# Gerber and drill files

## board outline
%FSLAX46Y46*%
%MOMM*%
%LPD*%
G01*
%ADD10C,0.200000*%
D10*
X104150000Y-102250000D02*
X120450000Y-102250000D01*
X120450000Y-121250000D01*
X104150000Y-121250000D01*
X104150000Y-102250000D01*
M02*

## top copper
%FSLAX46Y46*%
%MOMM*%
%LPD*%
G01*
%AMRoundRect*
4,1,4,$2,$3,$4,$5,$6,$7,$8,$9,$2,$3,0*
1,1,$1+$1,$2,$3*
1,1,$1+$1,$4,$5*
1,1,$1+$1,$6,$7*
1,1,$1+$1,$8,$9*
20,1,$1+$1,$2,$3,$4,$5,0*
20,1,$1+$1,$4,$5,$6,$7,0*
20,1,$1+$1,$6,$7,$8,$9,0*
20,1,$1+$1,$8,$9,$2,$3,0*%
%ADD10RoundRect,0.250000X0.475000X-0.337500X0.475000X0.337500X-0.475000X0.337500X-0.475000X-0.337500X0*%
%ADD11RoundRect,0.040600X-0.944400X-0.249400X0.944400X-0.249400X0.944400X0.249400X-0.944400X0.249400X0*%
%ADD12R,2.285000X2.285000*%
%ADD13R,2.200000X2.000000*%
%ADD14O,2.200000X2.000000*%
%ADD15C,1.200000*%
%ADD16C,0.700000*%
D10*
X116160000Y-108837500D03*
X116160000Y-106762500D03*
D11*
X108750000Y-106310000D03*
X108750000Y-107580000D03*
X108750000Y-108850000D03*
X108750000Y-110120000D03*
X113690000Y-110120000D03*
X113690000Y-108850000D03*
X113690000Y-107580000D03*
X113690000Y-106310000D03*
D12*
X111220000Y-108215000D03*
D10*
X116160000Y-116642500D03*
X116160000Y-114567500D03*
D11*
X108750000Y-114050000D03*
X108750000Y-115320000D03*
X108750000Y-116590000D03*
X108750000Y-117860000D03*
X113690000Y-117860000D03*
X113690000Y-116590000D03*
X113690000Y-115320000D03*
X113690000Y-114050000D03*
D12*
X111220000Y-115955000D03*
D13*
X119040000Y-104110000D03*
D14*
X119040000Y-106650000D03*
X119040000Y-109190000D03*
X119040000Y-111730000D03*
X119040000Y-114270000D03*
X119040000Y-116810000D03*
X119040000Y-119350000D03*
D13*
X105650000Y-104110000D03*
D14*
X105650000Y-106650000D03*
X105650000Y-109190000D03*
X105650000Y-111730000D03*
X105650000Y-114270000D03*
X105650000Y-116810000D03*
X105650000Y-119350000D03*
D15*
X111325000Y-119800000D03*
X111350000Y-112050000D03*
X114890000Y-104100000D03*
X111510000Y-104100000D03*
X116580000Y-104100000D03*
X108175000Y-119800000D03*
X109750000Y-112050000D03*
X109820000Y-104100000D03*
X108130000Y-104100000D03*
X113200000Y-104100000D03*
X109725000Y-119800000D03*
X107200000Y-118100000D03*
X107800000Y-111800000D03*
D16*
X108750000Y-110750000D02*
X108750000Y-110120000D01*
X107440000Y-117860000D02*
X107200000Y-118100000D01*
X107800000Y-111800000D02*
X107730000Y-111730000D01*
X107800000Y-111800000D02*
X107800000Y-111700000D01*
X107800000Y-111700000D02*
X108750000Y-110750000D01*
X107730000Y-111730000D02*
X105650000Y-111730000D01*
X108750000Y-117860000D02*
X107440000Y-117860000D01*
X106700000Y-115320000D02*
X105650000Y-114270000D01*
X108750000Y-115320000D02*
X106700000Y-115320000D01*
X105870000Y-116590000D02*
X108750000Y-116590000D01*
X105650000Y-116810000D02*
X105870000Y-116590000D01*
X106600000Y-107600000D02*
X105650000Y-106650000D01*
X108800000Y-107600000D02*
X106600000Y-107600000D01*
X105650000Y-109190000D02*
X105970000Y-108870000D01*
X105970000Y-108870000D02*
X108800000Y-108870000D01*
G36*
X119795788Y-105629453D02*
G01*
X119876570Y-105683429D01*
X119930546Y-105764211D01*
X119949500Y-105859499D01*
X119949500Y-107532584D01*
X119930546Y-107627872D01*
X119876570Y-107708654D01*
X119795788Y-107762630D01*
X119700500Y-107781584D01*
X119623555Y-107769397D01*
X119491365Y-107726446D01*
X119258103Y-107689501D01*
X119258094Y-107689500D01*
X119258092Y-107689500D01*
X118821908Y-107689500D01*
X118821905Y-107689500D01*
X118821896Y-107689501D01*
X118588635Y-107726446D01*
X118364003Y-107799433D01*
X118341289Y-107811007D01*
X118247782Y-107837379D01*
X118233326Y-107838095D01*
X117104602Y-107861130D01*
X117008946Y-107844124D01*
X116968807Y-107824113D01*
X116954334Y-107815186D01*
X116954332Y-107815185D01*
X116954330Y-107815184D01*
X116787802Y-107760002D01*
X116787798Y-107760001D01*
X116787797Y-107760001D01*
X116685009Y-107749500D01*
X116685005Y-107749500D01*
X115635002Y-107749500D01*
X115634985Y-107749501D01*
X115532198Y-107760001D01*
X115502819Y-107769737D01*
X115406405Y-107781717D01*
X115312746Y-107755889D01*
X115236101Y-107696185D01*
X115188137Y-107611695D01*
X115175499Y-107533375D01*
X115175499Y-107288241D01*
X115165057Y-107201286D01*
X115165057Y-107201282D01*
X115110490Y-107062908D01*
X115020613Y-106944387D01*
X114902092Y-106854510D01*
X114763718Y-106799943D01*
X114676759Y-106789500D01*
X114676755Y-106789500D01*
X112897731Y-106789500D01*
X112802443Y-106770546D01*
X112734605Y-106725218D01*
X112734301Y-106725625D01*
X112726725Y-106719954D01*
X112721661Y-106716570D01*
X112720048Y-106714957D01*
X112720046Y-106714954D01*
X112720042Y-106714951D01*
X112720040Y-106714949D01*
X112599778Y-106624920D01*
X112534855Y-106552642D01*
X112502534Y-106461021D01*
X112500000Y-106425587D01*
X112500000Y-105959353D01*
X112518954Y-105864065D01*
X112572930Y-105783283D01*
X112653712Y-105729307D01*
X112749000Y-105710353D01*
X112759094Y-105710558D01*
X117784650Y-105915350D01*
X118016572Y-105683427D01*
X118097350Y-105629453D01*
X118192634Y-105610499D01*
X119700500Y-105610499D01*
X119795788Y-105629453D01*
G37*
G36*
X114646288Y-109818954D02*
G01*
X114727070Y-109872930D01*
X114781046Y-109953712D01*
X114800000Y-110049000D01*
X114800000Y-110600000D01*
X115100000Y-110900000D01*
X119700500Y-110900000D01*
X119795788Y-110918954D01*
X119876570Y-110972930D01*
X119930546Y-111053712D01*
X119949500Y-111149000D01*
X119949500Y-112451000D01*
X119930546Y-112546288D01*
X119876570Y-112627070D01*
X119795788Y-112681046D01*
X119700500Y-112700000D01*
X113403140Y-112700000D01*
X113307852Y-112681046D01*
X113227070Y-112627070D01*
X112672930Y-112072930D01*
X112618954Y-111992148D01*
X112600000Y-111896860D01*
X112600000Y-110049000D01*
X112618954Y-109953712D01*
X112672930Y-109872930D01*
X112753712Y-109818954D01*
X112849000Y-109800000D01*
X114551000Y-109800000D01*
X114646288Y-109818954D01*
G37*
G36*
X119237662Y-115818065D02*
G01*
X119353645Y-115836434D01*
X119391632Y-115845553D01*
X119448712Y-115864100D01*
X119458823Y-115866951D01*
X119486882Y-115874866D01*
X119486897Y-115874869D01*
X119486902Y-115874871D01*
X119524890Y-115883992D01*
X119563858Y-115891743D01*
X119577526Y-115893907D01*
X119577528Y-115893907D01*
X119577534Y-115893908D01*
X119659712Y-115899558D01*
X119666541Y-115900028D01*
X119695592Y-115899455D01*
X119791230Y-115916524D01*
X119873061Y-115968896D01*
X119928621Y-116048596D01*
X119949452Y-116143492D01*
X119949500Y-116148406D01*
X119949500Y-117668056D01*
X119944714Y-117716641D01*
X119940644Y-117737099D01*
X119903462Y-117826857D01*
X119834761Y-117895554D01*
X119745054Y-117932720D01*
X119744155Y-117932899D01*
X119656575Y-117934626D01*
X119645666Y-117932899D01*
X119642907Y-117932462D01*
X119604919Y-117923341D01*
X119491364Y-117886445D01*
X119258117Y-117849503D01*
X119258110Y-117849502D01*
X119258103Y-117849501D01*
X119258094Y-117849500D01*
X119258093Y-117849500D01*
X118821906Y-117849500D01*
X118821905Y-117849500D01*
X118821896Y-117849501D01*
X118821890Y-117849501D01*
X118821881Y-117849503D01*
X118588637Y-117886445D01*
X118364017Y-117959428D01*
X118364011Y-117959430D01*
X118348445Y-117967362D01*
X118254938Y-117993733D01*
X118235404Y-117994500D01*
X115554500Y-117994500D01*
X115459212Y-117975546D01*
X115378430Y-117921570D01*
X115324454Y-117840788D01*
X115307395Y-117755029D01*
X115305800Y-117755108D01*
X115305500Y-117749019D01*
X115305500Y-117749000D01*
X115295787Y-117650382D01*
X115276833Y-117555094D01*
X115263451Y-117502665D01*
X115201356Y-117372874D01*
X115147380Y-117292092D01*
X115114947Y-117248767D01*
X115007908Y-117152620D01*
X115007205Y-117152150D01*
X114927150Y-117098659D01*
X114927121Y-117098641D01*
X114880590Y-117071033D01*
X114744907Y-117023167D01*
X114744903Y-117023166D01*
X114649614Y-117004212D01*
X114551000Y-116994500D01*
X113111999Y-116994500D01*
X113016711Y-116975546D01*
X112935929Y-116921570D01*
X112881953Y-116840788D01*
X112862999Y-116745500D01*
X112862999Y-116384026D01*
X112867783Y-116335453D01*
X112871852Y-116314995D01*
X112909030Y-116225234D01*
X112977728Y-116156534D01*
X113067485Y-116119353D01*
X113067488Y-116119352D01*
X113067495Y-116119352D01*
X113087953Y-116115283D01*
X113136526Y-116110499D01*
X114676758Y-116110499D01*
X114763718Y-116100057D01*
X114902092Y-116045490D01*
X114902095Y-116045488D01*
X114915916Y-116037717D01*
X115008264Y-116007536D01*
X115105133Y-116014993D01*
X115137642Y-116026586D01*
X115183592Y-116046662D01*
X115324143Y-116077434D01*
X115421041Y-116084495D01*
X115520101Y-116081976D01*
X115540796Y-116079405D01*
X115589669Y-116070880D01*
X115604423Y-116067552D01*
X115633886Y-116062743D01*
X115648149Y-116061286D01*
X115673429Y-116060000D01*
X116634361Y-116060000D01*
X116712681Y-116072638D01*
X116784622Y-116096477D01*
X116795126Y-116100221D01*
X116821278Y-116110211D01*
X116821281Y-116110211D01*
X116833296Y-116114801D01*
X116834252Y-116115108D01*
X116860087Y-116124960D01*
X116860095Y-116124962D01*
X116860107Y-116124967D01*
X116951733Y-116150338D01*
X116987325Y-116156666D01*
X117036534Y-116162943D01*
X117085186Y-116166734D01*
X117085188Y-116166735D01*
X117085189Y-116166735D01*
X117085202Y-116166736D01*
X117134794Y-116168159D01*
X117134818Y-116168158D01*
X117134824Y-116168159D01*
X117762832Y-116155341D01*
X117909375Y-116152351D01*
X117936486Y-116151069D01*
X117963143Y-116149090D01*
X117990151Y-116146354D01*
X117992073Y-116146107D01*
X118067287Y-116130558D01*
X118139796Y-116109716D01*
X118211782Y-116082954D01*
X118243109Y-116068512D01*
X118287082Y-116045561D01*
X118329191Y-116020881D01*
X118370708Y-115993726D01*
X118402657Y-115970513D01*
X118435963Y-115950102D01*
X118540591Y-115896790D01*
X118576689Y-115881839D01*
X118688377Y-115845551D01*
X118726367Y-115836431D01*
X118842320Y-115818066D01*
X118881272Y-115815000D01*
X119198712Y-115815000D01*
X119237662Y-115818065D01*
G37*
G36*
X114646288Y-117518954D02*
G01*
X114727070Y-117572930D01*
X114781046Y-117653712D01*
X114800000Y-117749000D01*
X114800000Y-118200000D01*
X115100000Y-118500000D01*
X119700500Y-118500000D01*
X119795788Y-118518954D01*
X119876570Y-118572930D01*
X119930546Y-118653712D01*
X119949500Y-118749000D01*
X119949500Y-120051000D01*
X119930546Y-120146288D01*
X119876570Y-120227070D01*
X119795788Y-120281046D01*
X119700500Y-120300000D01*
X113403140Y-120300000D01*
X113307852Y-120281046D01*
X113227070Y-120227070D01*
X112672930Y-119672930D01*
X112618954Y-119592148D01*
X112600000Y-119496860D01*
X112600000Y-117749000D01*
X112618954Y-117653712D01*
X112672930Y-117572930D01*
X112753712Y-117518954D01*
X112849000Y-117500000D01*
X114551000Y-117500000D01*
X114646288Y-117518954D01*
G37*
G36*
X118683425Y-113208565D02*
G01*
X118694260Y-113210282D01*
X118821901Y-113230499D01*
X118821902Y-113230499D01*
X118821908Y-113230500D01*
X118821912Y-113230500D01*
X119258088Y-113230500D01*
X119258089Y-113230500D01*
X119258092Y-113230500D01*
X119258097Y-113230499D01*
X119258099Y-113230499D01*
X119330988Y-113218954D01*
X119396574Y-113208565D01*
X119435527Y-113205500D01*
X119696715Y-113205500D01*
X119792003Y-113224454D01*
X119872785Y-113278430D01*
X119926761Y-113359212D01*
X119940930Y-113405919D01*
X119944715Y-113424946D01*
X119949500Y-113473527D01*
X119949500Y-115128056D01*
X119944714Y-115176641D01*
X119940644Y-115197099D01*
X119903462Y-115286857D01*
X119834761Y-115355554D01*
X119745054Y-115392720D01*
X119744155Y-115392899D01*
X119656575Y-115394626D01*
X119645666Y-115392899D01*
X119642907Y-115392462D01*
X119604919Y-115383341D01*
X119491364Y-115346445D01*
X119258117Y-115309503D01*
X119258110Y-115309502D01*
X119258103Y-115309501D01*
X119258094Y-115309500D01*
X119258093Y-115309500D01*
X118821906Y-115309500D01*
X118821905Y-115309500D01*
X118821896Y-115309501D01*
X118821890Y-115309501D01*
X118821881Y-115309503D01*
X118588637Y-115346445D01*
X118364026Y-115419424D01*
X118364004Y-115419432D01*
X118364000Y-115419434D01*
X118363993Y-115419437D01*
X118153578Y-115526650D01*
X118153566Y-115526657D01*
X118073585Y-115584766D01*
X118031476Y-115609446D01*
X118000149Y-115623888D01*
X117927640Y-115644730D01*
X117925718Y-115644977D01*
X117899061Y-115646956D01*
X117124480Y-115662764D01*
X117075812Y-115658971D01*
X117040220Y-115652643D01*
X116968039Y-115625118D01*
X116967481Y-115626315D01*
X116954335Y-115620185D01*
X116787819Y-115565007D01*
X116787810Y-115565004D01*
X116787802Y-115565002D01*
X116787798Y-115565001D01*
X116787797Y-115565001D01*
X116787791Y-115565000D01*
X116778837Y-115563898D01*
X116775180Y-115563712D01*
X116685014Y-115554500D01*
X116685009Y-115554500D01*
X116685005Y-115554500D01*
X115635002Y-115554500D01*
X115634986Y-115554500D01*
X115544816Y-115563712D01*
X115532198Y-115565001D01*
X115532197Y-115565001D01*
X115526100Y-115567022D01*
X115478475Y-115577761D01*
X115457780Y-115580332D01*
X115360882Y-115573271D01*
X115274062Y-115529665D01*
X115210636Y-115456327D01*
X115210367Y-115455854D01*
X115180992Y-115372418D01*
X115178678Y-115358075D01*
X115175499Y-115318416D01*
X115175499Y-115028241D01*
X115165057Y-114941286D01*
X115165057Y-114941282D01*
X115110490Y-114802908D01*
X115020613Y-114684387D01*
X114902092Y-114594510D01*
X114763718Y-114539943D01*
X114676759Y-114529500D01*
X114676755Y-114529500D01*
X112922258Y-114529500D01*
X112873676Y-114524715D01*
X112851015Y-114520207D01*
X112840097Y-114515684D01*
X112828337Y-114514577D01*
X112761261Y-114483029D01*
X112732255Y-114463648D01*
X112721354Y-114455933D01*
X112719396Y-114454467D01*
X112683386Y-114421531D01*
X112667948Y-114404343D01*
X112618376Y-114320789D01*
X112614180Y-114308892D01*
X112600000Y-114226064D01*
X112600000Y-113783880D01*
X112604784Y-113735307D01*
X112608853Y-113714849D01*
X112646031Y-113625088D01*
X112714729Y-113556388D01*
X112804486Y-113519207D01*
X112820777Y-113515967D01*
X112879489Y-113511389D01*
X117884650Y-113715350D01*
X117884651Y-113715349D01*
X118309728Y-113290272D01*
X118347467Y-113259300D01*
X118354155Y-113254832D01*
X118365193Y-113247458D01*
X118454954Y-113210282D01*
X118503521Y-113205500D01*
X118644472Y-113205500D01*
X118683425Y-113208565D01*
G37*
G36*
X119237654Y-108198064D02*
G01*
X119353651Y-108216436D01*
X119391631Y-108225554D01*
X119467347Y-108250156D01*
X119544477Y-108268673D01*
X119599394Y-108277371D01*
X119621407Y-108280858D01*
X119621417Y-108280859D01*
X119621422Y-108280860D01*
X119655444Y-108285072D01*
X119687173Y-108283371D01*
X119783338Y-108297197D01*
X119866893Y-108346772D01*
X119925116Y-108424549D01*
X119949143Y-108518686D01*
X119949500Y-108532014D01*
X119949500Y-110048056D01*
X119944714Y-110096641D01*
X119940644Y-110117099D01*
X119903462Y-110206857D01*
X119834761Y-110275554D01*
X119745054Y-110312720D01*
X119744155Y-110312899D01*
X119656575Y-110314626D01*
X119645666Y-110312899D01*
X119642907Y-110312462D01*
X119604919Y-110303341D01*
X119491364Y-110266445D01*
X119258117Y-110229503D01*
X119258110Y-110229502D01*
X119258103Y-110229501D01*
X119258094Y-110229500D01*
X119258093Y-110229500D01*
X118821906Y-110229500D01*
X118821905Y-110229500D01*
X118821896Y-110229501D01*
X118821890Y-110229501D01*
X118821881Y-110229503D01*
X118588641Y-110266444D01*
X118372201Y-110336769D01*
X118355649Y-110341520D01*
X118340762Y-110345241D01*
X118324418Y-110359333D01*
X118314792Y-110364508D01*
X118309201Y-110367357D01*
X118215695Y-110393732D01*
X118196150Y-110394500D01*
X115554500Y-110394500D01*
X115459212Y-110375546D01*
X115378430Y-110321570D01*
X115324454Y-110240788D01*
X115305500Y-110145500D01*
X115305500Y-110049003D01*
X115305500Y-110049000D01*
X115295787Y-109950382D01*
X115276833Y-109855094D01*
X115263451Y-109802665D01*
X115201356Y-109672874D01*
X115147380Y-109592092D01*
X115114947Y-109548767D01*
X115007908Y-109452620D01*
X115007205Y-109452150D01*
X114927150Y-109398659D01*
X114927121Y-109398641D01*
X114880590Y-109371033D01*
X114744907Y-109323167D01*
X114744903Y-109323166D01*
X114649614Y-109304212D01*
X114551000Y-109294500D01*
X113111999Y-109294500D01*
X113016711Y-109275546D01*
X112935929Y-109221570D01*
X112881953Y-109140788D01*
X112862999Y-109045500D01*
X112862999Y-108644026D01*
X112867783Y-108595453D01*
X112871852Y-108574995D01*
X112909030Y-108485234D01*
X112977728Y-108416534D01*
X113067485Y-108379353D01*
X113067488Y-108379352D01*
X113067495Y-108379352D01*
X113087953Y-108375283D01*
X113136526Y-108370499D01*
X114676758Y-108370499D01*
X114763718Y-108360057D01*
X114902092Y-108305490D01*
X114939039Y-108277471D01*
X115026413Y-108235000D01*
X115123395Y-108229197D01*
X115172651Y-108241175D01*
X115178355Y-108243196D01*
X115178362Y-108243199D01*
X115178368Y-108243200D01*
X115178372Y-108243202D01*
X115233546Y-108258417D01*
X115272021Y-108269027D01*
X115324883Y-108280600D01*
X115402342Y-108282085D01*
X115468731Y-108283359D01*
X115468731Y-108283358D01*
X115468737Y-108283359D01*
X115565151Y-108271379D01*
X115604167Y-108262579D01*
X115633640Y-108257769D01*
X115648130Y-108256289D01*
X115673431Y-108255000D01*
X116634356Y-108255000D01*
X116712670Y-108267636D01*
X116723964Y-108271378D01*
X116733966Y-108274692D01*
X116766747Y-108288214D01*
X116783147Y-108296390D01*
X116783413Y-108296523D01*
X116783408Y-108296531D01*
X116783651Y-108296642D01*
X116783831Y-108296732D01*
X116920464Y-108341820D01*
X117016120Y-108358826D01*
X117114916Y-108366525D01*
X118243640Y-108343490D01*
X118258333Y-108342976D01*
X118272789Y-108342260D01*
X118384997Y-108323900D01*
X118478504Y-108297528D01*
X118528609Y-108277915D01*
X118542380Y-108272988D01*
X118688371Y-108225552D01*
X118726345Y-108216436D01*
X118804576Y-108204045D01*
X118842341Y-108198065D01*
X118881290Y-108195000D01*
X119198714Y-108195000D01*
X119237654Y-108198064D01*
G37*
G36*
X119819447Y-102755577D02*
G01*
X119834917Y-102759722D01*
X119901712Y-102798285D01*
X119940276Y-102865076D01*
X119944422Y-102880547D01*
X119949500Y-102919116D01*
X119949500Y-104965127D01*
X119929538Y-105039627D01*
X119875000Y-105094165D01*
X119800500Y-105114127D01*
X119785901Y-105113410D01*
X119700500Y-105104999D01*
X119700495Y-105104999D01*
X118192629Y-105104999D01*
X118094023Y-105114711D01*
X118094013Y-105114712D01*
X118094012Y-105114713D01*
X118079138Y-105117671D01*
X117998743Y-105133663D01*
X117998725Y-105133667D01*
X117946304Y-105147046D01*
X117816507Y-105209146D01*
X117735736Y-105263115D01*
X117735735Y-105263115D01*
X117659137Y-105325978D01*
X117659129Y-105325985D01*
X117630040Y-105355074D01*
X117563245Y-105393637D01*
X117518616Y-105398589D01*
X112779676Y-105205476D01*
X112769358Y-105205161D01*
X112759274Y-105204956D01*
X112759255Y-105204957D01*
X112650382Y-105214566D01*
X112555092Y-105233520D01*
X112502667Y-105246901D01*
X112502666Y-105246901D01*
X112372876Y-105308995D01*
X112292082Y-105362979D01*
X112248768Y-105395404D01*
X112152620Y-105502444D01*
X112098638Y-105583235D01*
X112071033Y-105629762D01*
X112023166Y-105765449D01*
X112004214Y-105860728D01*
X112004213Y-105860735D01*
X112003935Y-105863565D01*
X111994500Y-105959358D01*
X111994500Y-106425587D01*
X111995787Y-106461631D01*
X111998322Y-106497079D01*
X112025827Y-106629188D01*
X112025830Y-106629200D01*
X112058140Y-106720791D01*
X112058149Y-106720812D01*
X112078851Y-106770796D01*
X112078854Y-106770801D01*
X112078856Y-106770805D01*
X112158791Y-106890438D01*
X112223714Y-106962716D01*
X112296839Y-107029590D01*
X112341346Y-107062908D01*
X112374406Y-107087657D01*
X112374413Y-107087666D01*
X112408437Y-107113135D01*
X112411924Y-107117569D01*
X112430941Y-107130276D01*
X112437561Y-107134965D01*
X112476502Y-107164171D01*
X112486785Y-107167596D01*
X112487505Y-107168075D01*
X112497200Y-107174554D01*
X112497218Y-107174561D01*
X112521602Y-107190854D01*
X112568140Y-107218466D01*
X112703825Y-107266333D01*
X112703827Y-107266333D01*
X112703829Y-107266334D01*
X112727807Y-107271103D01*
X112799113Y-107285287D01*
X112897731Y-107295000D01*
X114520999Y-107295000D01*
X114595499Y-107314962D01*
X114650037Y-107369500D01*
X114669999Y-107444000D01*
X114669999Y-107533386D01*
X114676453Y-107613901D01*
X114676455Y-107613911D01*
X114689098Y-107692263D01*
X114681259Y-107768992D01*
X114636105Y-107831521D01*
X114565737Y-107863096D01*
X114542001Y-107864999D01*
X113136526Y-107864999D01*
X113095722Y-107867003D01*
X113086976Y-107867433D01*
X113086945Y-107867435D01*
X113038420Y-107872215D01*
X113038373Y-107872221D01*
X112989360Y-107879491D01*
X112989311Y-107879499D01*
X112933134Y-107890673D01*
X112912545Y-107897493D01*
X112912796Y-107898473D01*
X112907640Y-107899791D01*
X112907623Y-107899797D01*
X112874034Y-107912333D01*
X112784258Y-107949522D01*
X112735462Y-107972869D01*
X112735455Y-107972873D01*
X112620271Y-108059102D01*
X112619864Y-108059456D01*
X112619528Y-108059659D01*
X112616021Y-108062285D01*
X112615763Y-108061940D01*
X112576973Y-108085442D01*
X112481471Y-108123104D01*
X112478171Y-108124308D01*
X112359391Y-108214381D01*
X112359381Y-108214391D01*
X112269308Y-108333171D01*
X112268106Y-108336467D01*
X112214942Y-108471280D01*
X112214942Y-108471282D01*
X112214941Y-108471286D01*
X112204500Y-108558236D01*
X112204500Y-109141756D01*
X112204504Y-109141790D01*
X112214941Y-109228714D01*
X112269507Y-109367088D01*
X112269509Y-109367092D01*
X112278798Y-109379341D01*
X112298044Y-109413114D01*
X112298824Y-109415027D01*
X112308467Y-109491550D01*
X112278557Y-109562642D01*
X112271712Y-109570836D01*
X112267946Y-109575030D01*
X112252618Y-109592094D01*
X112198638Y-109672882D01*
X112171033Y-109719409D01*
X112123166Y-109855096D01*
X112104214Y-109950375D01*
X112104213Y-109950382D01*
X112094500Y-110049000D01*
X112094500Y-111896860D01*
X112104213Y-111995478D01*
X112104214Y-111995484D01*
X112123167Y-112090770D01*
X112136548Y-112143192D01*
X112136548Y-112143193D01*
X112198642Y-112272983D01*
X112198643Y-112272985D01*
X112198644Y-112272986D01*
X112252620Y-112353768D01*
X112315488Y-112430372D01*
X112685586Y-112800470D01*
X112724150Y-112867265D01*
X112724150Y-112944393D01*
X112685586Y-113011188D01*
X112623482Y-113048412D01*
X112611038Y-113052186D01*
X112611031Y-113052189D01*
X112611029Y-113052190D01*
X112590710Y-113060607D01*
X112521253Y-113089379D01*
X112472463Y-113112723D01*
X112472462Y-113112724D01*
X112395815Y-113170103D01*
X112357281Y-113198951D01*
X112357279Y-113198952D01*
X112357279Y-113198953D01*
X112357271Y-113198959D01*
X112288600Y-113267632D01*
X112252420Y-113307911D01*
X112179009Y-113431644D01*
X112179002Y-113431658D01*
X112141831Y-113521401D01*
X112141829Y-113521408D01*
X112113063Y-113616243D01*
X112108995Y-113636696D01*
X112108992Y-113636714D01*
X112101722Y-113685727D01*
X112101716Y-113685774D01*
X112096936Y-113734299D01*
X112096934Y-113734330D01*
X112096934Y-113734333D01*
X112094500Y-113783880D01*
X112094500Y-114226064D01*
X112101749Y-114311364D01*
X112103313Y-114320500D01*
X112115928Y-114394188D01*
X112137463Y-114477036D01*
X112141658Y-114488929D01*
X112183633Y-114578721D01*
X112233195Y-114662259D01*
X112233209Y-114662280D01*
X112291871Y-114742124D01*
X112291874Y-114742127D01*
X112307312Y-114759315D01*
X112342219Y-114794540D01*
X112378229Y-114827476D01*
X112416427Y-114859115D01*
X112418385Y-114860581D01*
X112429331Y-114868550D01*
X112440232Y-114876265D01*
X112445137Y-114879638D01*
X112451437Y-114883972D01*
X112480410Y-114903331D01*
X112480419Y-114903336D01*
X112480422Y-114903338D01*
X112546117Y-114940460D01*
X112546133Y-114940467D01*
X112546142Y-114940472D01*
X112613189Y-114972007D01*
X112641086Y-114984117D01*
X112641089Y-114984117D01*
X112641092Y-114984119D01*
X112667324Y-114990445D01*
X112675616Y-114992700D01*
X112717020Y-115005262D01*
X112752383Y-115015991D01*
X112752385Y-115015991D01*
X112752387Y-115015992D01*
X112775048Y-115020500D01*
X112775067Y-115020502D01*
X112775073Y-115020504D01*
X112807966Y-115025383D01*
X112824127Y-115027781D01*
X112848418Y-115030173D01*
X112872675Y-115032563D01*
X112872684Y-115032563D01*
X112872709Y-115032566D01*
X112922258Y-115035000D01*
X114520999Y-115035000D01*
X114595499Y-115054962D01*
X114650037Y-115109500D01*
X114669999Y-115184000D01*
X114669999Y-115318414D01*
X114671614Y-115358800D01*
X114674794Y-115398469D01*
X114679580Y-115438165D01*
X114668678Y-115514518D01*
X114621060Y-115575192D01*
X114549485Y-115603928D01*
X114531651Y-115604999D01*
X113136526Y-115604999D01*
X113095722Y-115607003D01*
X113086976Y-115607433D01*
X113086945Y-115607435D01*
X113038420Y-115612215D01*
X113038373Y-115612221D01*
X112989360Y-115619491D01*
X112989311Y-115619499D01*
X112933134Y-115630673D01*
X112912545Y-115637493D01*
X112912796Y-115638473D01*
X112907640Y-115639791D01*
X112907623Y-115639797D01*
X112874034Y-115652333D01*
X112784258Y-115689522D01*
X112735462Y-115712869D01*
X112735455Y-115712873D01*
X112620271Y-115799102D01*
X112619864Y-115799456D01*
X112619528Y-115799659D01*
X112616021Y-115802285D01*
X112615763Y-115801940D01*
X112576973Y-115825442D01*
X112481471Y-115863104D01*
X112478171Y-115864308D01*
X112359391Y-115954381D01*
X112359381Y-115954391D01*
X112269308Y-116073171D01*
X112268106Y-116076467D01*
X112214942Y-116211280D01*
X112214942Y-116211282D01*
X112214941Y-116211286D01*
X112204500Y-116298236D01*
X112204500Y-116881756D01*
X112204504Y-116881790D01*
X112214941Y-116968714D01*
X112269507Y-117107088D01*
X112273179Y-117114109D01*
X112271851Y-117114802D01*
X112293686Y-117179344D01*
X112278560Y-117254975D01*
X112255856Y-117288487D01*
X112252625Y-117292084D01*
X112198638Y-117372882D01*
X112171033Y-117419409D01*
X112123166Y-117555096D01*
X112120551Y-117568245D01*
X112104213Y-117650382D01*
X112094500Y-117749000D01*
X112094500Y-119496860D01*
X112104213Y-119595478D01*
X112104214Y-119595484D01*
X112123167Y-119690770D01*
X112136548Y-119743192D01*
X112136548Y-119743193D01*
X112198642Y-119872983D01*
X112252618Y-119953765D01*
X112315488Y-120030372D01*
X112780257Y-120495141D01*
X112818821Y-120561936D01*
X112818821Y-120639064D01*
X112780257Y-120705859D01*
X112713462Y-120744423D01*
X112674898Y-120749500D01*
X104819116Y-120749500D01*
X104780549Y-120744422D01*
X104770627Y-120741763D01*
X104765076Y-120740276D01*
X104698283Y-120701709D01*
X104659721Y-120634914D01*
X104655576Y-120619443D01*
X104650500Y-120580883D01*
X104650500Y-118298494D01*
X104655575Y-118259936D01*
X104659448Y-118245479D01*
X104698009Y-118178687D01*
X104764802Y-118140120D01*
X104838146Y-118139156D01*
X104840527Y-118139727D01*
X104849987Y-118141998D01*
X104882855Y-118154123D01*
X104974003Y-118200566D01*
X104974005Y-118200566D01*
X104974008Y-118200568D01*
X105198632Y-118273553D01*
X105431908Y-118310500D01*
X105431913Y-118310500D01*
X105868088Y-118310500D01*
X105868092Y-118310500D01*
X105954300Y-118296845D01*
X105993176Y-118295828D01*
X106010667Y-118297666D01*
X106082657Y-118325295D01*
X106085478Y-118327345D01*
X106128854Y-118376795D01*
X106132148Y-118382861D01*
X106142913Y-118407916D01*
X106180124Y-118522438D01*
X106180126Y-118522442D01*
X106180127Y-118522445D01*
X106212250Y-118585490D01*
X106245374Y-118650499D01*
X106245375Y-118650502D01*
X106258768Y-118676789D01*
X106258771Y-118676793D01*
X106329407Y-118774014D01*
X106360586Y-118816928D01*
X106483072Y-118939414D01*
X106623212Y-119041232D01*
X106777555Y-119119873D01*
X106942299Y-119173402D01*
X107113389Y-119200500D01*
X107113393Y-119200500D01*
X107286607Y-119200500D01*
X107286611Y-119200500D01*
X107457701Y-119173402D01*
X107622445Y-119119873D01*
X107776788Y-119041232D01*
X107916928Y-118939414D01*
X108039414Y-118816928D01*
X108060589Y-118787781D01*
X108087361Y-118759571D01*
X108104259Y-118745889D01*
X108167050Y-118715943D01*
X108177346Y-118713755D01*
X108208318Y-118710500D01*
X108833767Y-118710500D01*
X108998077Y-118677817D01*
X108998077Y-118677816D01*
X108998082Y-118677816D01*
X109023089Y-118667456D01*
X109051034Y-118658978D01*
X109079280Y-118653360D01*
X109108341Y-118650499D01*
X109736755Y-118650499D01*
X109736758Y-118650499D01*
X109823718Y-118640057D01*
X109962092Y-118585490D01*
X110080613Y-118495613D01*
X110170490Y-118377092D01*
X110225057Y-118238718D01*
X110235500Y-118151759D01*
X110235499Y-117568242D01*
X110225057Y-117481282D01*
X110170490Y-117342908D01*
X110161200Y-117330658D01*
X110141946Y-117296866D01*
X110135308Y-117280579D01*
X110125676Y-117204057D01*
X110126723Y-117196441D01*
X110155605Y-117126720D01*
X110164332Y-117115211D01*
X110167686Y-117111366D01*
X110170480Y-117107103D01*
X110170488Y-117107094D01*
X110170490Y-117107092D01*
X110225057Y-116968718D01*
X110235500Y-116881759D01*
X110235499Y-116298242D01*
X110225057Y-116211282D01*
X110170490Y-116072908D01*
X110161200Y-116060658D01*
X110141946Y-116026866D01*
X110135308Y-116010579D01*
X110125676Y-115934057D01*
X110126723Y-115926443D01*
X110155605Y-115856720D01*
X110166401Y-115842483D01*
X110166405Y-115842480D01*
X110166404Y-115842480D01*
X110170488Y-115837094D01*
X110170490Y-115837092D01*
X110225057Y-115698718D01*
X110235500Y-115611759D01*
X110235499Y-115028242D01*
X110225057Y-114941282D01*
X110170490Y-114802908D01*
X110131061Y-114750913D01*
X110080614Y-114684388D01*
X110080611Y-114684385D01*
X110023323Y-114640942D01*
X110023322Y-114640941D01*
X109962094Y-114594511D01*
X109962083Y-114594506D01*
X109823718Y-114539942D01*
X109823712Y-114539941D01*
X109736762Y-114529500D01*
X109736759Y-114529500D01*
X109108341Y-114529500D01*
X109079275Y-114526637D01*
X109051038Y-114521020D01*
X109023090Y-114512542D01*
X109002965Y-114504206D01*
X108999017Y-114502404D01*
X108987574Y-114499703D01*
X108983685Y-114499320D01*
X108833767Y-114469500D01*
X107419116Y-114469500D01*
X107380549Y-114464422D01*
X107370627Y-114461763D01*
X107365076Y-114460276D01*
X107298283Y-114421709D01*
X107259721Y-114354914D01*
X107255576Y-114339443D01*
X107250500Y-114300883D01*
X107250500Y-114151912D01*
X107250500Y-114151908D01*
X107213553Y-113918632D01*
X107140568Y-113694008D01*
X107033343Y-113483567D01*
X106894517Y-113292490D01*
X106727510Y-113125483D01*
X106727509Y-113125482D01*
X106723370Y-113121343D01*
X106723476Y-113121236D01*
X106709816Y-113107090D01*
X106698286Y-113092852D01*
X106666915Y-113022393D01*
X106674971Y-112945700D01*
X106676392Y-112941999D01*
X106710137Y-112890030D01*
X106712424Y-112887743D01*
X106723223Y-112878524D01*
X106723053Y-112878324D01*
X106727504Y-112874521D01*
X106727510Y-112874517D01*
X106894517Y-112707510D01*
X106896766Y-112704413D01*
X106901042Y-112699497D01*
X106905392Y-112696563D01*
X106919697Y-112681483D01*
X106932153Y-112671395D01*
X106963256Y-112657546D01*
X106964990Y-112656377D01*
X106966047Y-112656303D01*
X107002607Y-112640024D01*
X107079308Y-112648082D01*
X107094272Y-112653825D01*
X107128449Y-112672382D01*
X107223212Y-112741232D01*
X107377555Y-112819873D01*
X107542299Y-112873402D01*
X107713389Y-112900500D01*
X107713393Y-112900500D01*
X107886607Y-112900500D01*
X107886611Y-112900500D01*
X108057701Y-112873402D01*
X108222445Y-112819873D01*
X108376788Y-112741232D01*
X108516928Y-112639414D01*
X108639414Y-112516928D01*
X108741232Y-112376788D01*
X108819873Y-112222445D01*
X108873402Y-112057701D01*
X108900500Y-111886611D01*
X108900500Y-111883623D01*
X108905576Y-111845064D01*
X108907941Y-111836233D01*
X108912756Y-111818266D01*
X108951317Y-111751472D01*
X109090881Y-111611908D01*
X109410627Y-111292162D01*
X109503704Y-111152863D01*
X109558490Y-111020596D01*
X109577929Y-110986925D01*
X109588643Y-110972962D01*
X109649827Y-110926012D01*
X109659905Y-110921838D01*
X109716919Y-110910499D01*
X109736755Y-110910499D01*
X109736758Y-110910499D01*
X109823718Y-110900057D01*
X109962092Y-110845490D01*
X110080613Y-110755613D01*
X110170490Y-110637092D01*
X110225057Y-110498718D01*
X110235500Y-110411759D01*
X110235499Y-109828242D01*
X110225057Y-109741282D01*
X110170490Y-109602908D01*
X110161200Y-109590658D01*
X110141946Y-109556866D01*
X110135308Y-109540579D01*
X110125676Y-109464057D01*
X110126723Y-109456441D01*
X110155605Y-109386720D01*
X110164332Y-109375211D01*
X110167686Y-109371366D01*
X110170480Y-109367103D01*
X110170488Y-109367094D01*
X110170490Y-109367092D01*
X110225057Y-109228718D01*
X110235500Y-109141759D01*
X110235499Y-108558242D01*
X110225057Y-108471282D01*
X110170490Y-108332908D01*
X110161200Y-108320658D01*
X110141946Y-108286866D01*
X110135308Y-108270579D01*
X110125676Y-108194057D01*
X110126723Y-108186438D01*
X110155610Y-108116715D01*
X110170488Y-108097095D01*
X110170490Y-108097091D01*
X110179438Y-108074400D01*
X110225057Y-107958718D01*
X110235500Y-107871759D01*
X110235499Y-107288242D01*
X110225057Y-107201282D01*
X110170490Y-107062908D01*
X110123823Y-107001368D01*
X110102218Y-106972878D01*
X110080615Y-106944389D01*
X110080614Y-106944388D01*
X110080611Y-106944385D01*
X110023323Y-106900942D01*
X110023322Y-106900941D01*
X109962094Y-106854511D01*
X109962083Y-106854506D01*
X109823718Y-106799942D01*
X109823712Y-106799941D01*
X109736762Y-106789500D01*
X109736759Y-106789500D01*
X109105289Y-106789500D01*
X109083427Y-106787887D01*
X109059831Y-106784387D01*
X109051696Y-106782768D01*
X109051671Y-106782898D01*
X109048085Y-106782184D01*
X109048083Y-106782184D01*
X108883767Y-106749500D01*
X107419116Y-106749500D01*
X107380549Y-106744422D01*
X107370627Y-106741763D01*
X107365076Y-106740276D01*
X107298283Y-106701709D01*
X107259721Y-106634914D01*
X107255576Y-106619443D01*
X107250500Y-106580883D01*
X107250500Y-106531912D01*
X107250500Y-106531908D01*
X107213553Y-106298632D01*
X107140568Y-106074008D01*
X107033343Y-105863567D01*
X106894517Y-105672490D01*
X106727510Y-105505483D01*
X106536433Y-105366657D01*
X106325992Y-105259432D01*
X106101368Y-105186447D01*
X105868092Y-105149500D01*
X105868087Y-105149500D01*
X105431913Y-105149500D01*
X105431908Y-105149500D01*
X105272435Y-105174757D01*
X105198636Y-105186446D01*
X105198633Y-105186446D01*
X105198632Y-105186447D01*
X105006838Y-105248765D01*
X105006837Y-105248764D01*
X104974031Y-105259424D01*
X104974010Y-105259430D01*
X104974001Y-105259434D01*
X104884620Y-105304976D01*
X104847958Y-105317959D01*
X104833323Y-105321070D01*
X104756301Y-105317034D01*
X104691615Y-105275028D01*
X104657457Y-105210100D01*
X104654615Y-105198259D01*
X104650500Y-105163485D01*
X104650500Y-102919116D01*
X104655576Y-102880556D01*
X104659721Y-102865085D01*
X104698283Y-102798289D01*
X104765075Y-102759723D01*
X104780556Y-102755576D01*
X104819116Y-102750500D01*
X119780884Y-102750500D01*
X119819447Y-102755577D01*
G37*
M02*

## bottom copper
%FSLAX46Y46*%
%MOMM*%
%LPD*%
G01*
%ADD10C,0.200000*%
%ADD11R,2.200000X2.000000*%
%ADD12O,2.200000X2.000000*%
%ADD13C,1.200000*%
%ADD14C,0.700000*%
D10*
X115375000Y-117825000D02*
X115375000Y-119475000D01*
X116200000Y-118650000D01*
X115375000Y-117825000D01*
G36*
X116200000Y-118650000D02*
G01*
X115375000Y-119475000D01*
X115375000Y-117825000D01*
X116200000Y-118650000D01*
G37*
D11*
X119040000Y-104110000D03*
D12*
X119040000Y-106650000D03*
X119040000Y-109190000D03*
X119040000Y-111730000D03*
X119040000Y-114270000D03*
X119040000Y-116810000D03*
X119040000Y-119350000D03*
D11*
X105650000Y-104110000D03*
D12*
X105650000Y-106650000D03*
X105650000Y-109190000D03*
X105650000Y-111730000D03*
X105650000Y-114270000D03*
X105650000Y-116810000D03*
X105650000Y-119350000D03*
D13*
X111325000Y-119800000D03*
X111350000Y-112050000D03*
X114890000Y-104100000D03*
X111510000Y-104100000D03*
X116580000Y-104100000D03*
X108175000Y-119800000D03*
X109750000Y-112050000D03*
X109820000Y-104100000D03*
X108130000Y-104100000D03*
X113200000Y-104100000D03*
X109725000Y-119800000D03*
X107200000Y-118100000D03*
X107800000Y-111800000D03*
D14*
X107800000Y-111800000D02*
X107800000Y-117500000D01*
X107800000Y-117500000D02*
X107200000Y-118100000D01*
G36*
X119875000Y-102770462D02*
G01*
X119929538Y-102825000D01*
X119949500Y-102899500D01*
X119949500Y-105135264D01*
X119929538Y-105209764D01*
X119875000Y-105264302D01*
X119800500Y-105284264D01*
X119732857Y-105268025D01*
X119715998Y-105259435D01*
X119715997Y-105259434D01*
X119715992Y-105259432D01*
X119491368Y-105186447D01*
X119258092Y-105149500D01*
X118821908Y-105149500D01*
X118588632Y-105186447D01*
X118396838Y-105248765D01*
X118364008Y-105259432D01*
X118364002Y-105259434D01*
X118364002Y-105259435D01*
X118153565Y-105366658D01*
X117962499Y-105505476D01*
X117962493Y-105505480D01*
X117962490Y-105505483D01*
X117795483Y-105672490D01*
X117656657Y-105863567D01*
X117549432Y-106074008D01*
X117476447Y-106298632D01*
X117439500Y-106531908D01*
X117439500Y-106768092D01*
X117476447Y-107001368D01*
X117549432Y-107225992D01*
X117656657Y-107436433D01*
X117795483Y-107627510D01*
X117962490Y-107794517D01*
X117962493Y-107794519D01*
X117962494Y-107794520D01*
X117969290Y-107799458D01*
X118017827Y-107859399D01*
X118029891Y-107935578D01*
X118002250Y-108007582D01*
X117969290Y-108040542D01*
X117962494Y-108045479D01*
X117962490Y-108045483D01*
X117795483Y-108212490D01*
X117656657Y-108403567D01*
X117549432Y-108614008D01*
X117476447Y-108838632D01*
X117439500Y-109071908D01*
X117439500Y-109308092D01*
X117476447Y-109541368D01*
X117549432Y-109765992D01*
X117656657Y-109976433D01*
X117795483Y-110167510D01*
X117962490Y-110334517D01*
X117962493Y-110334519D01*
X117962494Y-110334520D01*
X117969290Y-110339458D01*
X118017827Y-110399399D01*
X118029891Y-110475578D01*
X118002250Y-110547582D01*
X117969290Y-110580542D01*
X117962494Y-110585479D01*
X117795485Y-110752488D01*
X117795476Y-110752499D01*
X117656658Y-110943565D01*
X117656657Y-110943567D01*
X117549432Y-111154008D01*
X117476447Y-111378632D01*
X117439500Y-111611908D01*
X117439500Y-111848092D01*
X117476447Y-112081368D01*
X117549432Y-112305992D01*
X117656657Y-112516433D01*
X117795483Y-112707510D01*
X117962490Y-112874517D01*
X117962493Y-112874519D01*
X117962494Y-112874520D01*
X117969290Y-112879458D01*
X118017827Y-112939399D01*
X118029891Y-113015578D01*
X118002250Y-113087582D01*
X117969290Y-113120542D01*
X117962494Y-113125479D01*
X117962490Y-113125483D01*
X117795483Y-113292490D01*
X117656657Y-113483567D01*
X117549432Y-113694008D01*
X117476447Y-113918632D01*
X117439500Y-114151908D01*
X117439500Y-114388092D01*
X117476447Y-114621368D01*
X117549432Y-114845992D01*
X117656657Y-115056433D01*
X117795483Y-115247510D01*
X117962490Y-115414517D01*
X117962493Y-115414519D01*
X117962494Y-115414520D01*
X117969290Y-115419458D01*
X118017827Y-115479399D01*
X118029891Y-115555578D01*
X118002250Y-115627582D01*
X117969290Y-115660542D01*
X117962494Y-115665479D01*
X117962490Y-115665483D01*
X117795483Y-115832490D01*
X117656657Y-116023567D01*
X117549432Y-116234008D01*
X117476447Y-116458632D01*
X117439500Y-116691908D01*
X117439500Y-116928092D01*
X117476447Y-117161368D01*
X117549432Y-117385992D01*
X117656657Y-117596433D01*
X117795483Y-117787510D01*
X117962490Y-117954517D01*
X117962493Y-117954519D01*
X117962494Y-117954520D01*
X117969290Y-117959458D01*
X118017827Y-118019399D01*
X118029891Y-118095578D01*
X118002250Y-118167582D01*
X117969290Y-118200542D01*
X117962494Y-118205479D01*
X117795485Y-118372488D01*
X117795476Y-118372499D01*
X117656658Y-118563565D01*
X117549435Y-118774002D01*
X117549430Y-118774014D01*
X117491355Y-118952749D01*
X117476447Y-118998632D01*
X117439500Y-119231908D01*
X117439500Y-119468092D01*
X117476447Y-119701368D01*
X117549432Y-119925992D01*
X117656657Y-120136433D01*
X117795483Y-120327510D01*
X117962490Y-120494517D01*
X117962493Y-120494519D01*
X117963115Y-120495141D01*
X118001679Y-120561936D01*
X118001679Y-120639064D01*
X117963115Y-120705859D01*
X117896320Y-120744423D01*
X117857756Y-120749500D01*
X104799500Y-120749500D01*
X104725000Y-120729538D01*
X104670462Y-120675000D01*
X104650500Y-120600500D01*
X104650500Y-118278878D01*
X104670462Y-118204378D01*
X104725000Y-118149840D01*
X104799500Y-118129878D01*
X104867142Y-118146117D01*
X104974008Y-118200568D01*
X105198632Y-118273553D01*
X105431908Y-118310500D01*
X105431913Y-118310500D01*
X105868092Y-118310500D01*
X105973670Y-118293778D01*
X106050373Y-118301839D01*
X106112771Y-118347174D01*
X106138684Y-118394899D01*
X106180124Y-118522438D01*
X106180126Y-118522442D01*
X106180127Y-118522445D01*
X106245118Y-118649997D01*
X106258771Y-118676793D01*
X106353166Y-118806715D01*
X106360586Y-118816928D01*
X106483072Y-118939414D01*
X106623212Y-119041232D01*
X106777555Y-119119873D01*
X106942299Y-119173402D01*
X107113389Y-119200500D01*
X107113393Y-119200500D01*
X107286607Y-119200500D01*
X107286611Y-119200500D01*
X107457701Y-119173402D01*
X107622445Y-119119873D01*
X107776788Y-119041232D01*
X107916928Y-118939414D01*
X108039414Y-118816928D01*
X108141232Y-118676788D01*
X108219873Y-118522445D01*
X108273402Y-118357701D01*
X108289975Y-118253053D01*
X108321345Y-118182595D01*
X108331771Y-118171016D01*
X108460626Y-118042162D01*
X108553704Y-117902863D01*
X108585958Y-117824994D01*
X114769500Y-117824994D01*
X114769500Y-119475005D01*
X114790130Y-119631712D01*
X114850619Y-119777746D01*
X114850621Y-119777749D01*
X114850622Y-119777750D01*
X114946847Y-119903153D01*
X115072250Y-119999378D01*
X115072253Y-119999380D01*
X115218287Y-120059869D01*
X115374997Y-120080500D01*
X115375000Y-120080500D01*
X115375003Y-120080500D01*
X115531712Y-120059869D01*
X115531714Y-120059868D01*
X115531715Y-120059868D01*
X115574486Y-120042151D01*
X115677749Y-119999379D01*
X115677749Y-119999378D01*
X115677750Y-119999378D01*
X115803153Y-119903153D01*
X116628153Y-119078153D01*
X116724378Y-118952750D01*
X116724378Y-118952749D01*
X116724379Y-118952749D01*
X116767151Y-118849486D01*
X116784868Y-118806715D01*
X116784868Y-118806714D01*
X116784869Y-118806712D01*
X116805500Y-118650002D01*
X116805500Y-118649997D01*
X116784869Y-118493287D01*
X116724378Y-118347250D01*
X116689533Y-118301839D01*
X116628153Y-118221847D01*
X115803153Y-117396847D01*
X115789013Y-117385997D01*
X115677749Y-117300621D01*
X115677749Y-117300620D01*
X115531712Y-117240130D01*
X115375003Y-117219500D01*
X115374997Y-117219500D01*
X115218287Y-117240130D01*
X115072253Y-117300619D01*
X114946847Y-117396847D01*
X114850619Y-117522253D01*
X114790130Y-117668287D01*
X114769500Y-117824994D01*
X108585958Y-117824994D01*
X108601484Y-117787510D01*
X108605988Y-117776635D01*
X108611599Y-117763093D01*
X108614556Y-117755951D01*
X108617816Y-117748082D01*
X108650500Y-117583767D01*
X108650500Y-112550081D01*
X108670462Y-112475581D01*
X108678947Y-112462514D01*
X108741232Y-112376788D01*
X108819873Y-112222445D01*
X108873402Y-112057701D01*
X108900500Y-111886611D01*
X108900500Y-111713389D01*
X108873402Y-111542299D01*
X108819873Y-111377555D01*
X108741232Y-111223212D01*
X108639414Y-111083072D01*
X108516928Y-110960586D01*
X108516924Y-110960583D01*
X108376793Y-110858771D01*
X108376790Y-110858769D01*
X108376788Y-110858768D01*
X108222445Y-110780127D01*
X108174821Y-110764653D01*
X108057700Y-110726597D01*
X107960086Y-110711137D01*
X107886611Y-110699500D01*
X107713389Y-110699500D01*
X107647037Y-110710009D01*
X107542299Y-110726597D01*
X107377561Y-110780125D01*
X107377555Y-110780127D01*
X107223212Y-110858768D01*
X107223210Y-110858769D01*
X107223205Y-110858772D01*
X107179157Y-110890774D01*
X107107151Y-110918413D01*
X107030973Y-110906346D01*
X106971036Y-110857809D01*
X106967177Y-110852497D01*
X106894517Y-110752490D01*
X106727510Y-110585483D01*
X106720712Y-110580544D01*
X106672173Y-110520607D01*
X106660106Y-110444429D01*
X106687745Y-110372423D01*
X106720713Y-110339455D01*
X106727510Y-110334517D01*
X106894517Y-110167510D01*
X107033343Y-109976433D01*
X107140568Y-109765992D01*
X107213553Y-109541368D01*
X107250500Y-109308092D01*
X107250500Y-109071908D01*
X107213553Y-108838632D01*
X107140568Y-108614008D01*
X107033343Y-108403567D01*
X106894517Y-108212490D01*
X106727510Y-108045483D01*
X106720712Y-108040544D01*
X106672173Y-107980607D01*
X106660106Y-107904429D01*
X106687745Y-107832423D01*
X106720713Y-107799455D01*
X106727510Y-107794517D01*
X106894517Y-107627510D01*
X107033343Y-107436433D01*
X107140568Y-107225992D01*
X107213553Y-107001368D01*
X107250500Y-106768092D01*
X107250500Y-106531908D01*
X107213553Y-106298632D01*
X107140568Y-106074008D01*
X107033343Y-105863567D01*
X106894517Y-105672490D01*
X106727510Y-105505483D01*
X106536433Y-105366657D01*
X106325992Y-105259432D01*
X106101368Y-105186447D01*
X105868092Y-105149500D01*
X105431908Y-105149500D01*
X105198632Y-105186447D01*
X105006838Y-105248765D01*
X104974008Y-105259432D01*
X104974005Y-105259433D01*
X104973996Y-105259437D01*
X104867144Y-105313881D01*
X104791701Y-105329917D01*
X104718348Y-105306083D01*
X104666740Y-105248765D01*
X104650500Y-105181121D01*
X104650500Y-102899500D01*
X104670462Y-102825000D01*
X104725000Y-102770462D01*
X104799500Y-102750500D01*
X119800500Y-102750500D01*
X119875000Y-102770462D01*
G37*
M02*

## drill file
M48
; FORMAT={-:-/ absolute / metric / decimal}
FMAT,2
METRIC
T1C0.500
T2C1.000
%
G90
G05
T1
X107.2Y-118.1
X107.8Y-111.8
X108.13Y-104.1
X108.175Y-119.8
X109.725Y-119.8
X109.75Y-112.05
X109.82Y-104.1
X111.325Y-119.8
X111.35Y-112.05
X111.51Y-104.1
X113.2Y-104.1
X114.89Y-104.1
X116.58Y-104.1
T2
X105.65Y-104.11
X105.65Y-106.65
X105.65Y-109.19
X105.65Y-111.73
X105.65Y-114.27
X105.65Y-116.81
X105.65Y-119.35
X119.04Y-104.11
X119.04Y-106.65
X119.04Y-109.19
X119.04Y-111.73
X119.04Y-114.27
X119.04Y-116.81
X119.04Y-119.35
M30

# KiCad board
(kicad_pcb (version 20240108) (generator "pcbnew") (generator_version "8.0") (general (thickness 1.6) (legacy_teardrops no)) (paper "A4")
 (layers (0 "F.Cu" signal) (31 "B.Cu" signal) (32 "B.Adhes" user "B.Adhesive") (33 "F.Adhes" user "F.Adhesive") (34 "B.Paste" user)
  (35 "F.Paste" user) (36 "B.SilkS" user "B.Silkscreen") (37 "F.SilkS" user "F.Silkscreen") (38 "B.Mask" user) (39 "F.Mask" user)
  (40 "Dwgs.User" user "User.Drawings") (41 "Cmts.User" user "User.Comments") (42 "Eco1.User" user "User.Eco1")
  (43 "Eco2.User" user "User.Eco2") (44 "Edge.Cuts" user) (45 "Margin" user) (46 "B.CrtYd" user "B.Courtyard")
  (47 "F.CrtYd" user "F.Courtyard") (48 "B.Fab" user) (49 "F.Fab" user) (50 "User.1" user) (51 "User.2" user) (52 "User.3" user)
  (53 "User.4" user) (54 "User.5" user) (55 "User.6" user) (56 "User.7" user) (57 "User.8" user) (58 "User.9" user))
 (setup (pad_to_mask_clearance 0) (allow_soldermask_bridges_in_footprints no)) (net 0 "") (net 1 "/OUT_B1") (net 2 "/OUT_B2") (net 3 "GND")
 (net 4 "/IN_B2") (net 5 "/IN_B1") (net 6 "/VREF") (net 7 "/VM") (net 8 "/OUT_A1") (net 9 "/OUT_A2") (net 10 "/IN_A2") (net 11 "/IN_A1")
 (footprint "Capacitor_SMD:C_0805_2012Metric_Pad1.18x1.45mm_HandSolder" (layer "F.Cu") (at 116.16 107.8 90)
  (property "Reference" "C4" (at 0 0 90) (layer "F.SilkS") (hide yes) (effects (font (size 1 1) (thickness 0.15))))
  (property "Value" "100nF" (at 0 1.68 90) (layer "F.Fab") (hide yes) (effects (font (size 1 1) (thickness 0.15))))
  (pad "1" smd roundrect (at -1.0375 0 90) (size 1.175 1.45) (layers "F.Cu" "F.Paste" "F.Mask") (roundrect_rratio 0.212766)
   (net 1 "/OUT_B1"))
  (pad "2" smd roundrect (at 1.0375 0 90) (size 1.175 1.45) (layers "F.Cu" "F.Paste" "F.Mask") (roundrect_rratio 0.212766) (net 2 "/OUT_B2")))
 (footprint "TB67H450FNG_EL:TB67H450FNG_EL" (layer "F.Cu") (at 111.22 108.215)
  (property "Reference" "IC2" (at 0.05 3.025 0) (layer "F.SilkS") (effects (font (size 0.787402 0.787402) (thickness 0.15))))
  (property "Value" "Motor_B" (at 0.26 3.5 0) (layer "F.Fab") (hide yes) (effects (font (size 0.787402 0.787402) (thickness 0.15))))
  (pad "1" smd roundrect (at -2.47 -1.905) (size 1.97 0.58) (layers "F.Cu" "F.Paste" "F.Mask") (roundrect_rratio 0.07) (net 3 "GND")
   (solder_mask_margin 0.102))
  (pad "2" smd roundrect (at -2.47 -0.635) (size 1.97 0.58) (layers "F.Cu" "F.Paste" "F.Mask") (roundrect_rratio 0.07) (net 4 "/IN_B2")
   (solder_mask_margin 0.102))
  (pad "3" smd roundrect (at -2.47 0.635) (size 1.97 0.58) (layers "F.Cu" "F.Paste" "F.Mask") (roundrect_rratio 0.07) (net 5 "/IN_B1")
   (solder_mask_margin 0.102))
  (pad "4" smd roundrect (at -2.47 1.905) (size 1.97 0.58) (layers "F.Cu" "F.Paste" "F.Mask") (roundrect_rratio 0.07) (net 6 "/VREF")
   (solder_mask_margin 0.102))
  (pad "5" smd roundrect (at 2.47 1.905) (size 1.97 0.58) (layers "F.Cu" "F.Paste" "F.Mask") (roundrect_rratio 0.07) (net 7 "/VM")
   (solder_mask_margin 0.102))
  (pad "6" smd roundrect (at 2.47 0.635) (size 1.97 0.58) (layers "F.Cu" "F.Paste" "F.Mask") (roundrect_rratio 0.07) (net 1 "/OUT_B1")
   (solder_mask_margin 0.102))
  (pad "7" smd roundrect (at 2.47 -0.635) (size 1.97 0.58) (layers "F.Cu" "F.Paste" "F.Mask") (roundrect_rratio 0.07) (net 3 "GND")
   (solder_mask_margin 0.102))
  (pad "8" smd roundrect (at 2.47 -1.905) (size 1.97 0.58) (layers "F.Cu" "F.Paste" "F.Mask") (roundrect_rratio 0.07) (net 2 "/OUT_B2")
   (solder_mask_margin 0.102))
  (pad "9" smd rect (at 0 0) (size 2.285 2.285) (layers "F.Cu" "F.Mask") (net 3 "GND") (solder_mask_margin 0.102)))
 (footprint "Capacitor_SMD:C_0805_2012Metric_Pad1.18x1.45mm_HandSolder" (layer "F.Cu") (at 116.16 115.605 90)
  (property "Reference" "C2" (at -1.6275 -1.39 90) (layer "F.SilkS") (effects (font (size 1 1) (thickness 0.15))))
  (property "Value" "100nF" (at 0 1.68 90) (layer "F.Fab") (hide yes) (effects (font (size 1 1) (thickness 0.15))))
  (pad "1" smd roundrect (at -1.0375 0 90) (size 1.175 1.45) (layers "F.Cu" "F.Paste" "F.Mask") (roundrect_rratio 0.212766)
   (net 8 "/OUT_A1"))
  (pad "2" smd roundrect (at 1.0375 0 90) (size 1.175 1.45) (layers "F.Cu" "F.Paste" "F.Mask") (roundrect_rratio 0.212766) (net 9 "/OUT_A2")))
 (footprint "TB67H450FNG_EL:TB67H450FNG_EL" (layer "F.Cu") (at 111.22 115.955)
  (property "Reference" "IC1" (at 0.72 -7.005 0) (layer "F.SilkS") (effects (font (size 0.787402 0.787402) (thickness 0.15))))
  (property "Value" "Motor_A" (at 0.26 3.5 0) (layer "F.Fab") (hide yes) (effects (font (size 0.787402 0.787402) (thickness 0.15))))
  (pad "1" smd roundrect (at -2.47 -1.905) (size 1.97 0.58) (layers "F.Cu" "F.Paste" "F.Mask") (roundrect_rratio 0.07) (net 3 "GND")
   (solder_mask_margin 0.102))
  (pad "2" smd roundrect (at -2.47 -0.635) (size 1.97 0.58) (layers "F.Cu" "F.Paste" "F.Mask") (roundrect_rratio 0.07) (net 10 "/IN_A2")
   (solder_mask_margin 0.102))
  (pad "3" smd roundrect (at -2.47 0.635) (size 1.97 0.58) (layers "F.Cu" "F.Paste" "F.Mask") (roundrect_rratio 0.07) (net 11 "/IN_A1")
   (solder_mask_margin 0.102))
  (pad "4" smd roundrect (at -2.47 1.905) (size 1.97 0.58) (layers "F.Cu" "F.Paste" "F.Mask") (roundrect_rratio 0.07) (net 6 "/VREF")
   (solder_mask_margin 0.102))
  (pad "5" smd roundrect (at 2.47 1.905) (size 1.97 0.58) (layers "F.Cu" "F.Paste" "F.Mask") (roundrect_rratio 0.07) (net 7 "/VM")
   (solder_mask_margin 0.102))
  (pad "6" smd roundrect (at 2.47 0.635) (size 1.97 0.58) (layers "F.Cu" "F.Paste" "F.Mask") (roundrect_rratio 0.07) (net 8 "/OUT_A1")
   (solder_mask_margin 0.102))
  (pad "7" smd roundrect (at 2.47 -0.635) (size 1.97 0.58) (layers "F.Cu" "F.Paste" "F.Mask") (roundrect_rratio 0.07) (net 3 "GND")
   (solder_mask_margin 0.102))
  (pad "8" smd roundrect (at 2.47 -1.905) (size 1.97 0.58) (layers "F.Cu" "F.Paste" "F.Mask") (roundrect_rratio 0.07) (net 9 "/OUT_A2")
   (solder_mask_margin 0.102))
  (pad "9" smd rect (at 0 0) (size 2.285 2.285) (layers "F.Cu" "F.Mask") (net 3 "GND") (solder_mask_margin 0.102)))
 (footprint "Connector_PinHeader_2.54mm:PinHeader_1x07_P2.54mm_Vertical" (layer "B.Cu") (at 119.04 104.11 180)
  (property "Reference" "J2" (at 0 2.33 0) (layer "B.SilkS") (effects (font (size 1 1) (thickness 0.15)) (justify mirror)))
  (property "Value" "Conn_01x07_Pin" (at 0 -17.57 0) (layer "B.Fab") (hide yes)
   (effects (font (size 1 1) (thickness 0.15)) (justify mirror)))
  (pad "1" thru_hole rect (at 0 0 180) (size 2.2 2) (drill 1) (layers "*.Cu" "*.Mask") (remove_unused_layers no) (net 3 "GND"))
  (pad "2" thru_hole oval (at 0 -2.54 180) (size 2.2 2) (drill 1) (layers "*.Cu" "*.Mask") (remove_unused_layers no) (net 2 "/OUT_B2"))
  (pad "3" thru_hole oval (at 0 -5.08 180) (size 2.2 2) (drill 1) (layers "*.Cu" "*.Mask") (remove_unused_layers no) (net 1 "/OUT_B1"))
  (pad "4" thru_hole oval (at 0 -7.62 180) (size 2.2 2) (drill 1) (layers "*.Cu" "*.Mask") (remove_unused_layers no) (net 7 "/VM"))
  (pad "5" thru_hole oval (at 0 -10.16 180) (size 2.2 2) (drill 1) (layers "*.Cu" "*.Mask") (remove_unused_layers no) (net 9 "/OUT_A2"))
  (pad "6" thru_hole oval (at 0 -12.7 180) (size 2.2 2) (drill 1) (layers "*.Cu" "*.Mask") (remove_unused_layers no) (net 8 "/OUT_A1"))
  (pad "7" thru_hole oval (at 0 -15.24 180) (size 2.2 2) (drill 1) (layers "*.Cu" "*.Mask") (remove_unused_layers no) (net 7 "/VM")))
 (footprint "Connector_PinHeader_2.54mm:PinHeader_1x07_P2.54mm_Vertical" (layer "B.Cu") (at 105.65 104.11 180)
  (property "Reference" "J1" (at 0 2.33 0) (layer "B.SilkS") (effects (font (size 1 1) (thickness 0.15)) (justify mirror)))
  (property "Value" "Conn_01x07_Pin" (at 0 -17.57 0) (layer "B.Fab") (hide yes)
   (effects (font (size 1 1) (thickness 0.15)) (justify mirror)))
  (pad "1" thru_hole rect (at 0 0 180) (size 2.2 2) (drill 1) (layers "*.Cu" "*.Mask") (remove_unused_layers no) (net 3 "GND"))
  (pad "2" thru_hole oval (at 0 -2.54 180) (size 2.2 2) (drill 1) (layers "*.Cu" "*.Mask") (remove_unused_layers no) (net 4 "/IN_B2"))
  (pad "3" thru_hole oval (at 0 -5.08 180) (size 2.2 2) (drill 1) (layers "*.Cu" "*.Mask") (remove_unused_layers no) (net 5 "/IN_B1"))
  (pad "4" thru_hole oval (at 0 -7.62 180) (size 2.2 2) (drill 1) (layers "*.Cu" "*.Mask") (remove_unused_layers no) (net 6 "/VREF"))
  (pad "5" thru_hole oval (at 0 -10.16 180) (size 2.2 2) (drill 1) (layers "*.Cu" "*.Mask") (remove_unused_layers no) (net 10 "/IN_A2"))
  (pad "6" thru_hole oval (at 0 -12.7 180) (size 2.2 2) (drill 1) (layers "*.Cu" "*.Mask") (remove_unused_layers no) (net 11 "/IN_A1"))
  (pad "7" thru_hole oval (at 0 -15.24 180) (size 2.2 2) (drill 1) (layers "*.Cu" "*.Mask") (remove_unused_layers no) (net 3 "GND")))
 (gr_poly (pts (xy 115.375 117.825) (xy 115.375 119.475) (xy 116.2 118.65)) (stroke (width 0.2) (type solid)) (fill solid) (layer "B.Cu"))
 (gr_rect (start 104.15 102.25) (end 120.45 121.25) (stroke (width 0.2) (type default)) (fill none) (layer "Edge.Cuts"))
 (via (at 111.325 119.8) (size 1.2) (drill 0.5) (layers "F.Cu" "B.Cu") (free yes) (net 3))
 (via (at 111.35 112.05) (size 1.2) (drill 0.5) (layers "F.Cu" "B.Cu") (free yes) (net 3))
 (via (at 114.89 104.1) (size 1.2) (drill 0.5) (layers "F.Cu" "B.Cu") (free yes) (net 3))
 (via (at 111.51 104.1) (size 1.2) (drill 0.5) (layers "F.Cu" "B.Cu") (free yes) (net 3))
 (via (at 116.58 104.1) (size 1.2) (drill 0.5) (layers "F.Cu" "B.Cu") (free yes) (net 3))
 (via (at 108.175 119.8) (size 1.2) (drill 0.5) (layers "F.Cu" "B.Cu") (free yes) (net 3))
 (via (at 109.75 112.05) (size 1.2) (drill 0.5) (layers "F.Cu" "B.Cu") (free yes) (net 3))
 (via (at 109.82 104.1) (size 1.2) (drill 0.5) (layers "F.Cu" "B.Cu") (free yes) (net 3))
 (via (at 108.13 104.1) (size 1.2) (drill 0.5) (layers "F.Cu" "B.Cu") (free yes) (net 3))
 (via (at 113.2 104.1) (size 1.2) (drill 0.5) (layers "F.Cu" "B.Cu") (free yes) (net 3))
 (via (at 109.725 119.8) (size 1.2) (drill 0.5) (layers "F.Cu" "B.Cu") (free yes) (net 3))
 (segment (start 108.75 110.75) (end 108.75 110.12) (width 0.7) (layer "F.Cu") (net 6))
 (segment (start 107.44 117.86) (end 107.2 118.1) (width 0.7) (layer "F.Cu") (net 6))
 (segment (start 107.8 111.8) (end 107.73 111.73) (width 0.7) (layer "F.Cu") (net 6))
 (segment (start 107.8 111.8) (end 107.8 111.7) (width 0.7) (layer "F.Cu") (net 6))
 (segment (start 107.8 111.7) (end 108.75 110.75) (width 0.7) (layer "F.Cu") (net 6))
 (segment (start 107.73 111.73) (end 105.65 111.73) (width 0.7) (layer "F.Cu") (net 6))
 (segment (start 108.75 117.86) (end 107.44 117.86) (width 0.7) (layer "F.Cu") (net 6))
 (via (at 107.2 118.1) (size 1.2) (drill 0.5) (layers "F.Cu" "B.Cu") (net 6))
 (via (at 107.8 111.8) (size 1.2) (drill 0.5) (layers "F.Cu" "B.Cu") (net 6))
 (segment (start 107.8 111.8) (end 107.8 117.5) (width 0.7) (layer "B.Cu") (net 6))
 (segment (start 107.8 117.5) (end 107.2 118.1) (width 0.7) (layer "B.Cu") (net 6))
 (segment (start 106.7 115.32) (end 105.65 114.27) (width 0.7) (layer "F.Cu") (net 10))
 (segment (start 108.75 115.32) (end 106.7 115.32) (width 0.7) (layer "F.Cu") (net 10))
 (segment (start 105.87 116.59) (end 108.75 116.59) (width 0.7) (layer "F.Cu") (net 11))
 (segment (start 105.65 116.81) (end 105.87 116.59) (width 0.7) (layer "F.Cu") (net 11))
 (segment (start 106.6 107.6) (end 105.65 106.65) (width 0.7) (layer "F.Cu") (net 4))
 (segment (start 108.8 107.6) (end 106.6 107.6) (width 0.7) (layer "F.Cu") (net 4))
 (segment (start 105.65 109.19) (end 105.97 108.87) (width 0.7) (layer "F.Cu") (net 5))
 (segment (start 105.97 108.87) (end 108.8 108.87) (width 0.7) (layer "F.Cu") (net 5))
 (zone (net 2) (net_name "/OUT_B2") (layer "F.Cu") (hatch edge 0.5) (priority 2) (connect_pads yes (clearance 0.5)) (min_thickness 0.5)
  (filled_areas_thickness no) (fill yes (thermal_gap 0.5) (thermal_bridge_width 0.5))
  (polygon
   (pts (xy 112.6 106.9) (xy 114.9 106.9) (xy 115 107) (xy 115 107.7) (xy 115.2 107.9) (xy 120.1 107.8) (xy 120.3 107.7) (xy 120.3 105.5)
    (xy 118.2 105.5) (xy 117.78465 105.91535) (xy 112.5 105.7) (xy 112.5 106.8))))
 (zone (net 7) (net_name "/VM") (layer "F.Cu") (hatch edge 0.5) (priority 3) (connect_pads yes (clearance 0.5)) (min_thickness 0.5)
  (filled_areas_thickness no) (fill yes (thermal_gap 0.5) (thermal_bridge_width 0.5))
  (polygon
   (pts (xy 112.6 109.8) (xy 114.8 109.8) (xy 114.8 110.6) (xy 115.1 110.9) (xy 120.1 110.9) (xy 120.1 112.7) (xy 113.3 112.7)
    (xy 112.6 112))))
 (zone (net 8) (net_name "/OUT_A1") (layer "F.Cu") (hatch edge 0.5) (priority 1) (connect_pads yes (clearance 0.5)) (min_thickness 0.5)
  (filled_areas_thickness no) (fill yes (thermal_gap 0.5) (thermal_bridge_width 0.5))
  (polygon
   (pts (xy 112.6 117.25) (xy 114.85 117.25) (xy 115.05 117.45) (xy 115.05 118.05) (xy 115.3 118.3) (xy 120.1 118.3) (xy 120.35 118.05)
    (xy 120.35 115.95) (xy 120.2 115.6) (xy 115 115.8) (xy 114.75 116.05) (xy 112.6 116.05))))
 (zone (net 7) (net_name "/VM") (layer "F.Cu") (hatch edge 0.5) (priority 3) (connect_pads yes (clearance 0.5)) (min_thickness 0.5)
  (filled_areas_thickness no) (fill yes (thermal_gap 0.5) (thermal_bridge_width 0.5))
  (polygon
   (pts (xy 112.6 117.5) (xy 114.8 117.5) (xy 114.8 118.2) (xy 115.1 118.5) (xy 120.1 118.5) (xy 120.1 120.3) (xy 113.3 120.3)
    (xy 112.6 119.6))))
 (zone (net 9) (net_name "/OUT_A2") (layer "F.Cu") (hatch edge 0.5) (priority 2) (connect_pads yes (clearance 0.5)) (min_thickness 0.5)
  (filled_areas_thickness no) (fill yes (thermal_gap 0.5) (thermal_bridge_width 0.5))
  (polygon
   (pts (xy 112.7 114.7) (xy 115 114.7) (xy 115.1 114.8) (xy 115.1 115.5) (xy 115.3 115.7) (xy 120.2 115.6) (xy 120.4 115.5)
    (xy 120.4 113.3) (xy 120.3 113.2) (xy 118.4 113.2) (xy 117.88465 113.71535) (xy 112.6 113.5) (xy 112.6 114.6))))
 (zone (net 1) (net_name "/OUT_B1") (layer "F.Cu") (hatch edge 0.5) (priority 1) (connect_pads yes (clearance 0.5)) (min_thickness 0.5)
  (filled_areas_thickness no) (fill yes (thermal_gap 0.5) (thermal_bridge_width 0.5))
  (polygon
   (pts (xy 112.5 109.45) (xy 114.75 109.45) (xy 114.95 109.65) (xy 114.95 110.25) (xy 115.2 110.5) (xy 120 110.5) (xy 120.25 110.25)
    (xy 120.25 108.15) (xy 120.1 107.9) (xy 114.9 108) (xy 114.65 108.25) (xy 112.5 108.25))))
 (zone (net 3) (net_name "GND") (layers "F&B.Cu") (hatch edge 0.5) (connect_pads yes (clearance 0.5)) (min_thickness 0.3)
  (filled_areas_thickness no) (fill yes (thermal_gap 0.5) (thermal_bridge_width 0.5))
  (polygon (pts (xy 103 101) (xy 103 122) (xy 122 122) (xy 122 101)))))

